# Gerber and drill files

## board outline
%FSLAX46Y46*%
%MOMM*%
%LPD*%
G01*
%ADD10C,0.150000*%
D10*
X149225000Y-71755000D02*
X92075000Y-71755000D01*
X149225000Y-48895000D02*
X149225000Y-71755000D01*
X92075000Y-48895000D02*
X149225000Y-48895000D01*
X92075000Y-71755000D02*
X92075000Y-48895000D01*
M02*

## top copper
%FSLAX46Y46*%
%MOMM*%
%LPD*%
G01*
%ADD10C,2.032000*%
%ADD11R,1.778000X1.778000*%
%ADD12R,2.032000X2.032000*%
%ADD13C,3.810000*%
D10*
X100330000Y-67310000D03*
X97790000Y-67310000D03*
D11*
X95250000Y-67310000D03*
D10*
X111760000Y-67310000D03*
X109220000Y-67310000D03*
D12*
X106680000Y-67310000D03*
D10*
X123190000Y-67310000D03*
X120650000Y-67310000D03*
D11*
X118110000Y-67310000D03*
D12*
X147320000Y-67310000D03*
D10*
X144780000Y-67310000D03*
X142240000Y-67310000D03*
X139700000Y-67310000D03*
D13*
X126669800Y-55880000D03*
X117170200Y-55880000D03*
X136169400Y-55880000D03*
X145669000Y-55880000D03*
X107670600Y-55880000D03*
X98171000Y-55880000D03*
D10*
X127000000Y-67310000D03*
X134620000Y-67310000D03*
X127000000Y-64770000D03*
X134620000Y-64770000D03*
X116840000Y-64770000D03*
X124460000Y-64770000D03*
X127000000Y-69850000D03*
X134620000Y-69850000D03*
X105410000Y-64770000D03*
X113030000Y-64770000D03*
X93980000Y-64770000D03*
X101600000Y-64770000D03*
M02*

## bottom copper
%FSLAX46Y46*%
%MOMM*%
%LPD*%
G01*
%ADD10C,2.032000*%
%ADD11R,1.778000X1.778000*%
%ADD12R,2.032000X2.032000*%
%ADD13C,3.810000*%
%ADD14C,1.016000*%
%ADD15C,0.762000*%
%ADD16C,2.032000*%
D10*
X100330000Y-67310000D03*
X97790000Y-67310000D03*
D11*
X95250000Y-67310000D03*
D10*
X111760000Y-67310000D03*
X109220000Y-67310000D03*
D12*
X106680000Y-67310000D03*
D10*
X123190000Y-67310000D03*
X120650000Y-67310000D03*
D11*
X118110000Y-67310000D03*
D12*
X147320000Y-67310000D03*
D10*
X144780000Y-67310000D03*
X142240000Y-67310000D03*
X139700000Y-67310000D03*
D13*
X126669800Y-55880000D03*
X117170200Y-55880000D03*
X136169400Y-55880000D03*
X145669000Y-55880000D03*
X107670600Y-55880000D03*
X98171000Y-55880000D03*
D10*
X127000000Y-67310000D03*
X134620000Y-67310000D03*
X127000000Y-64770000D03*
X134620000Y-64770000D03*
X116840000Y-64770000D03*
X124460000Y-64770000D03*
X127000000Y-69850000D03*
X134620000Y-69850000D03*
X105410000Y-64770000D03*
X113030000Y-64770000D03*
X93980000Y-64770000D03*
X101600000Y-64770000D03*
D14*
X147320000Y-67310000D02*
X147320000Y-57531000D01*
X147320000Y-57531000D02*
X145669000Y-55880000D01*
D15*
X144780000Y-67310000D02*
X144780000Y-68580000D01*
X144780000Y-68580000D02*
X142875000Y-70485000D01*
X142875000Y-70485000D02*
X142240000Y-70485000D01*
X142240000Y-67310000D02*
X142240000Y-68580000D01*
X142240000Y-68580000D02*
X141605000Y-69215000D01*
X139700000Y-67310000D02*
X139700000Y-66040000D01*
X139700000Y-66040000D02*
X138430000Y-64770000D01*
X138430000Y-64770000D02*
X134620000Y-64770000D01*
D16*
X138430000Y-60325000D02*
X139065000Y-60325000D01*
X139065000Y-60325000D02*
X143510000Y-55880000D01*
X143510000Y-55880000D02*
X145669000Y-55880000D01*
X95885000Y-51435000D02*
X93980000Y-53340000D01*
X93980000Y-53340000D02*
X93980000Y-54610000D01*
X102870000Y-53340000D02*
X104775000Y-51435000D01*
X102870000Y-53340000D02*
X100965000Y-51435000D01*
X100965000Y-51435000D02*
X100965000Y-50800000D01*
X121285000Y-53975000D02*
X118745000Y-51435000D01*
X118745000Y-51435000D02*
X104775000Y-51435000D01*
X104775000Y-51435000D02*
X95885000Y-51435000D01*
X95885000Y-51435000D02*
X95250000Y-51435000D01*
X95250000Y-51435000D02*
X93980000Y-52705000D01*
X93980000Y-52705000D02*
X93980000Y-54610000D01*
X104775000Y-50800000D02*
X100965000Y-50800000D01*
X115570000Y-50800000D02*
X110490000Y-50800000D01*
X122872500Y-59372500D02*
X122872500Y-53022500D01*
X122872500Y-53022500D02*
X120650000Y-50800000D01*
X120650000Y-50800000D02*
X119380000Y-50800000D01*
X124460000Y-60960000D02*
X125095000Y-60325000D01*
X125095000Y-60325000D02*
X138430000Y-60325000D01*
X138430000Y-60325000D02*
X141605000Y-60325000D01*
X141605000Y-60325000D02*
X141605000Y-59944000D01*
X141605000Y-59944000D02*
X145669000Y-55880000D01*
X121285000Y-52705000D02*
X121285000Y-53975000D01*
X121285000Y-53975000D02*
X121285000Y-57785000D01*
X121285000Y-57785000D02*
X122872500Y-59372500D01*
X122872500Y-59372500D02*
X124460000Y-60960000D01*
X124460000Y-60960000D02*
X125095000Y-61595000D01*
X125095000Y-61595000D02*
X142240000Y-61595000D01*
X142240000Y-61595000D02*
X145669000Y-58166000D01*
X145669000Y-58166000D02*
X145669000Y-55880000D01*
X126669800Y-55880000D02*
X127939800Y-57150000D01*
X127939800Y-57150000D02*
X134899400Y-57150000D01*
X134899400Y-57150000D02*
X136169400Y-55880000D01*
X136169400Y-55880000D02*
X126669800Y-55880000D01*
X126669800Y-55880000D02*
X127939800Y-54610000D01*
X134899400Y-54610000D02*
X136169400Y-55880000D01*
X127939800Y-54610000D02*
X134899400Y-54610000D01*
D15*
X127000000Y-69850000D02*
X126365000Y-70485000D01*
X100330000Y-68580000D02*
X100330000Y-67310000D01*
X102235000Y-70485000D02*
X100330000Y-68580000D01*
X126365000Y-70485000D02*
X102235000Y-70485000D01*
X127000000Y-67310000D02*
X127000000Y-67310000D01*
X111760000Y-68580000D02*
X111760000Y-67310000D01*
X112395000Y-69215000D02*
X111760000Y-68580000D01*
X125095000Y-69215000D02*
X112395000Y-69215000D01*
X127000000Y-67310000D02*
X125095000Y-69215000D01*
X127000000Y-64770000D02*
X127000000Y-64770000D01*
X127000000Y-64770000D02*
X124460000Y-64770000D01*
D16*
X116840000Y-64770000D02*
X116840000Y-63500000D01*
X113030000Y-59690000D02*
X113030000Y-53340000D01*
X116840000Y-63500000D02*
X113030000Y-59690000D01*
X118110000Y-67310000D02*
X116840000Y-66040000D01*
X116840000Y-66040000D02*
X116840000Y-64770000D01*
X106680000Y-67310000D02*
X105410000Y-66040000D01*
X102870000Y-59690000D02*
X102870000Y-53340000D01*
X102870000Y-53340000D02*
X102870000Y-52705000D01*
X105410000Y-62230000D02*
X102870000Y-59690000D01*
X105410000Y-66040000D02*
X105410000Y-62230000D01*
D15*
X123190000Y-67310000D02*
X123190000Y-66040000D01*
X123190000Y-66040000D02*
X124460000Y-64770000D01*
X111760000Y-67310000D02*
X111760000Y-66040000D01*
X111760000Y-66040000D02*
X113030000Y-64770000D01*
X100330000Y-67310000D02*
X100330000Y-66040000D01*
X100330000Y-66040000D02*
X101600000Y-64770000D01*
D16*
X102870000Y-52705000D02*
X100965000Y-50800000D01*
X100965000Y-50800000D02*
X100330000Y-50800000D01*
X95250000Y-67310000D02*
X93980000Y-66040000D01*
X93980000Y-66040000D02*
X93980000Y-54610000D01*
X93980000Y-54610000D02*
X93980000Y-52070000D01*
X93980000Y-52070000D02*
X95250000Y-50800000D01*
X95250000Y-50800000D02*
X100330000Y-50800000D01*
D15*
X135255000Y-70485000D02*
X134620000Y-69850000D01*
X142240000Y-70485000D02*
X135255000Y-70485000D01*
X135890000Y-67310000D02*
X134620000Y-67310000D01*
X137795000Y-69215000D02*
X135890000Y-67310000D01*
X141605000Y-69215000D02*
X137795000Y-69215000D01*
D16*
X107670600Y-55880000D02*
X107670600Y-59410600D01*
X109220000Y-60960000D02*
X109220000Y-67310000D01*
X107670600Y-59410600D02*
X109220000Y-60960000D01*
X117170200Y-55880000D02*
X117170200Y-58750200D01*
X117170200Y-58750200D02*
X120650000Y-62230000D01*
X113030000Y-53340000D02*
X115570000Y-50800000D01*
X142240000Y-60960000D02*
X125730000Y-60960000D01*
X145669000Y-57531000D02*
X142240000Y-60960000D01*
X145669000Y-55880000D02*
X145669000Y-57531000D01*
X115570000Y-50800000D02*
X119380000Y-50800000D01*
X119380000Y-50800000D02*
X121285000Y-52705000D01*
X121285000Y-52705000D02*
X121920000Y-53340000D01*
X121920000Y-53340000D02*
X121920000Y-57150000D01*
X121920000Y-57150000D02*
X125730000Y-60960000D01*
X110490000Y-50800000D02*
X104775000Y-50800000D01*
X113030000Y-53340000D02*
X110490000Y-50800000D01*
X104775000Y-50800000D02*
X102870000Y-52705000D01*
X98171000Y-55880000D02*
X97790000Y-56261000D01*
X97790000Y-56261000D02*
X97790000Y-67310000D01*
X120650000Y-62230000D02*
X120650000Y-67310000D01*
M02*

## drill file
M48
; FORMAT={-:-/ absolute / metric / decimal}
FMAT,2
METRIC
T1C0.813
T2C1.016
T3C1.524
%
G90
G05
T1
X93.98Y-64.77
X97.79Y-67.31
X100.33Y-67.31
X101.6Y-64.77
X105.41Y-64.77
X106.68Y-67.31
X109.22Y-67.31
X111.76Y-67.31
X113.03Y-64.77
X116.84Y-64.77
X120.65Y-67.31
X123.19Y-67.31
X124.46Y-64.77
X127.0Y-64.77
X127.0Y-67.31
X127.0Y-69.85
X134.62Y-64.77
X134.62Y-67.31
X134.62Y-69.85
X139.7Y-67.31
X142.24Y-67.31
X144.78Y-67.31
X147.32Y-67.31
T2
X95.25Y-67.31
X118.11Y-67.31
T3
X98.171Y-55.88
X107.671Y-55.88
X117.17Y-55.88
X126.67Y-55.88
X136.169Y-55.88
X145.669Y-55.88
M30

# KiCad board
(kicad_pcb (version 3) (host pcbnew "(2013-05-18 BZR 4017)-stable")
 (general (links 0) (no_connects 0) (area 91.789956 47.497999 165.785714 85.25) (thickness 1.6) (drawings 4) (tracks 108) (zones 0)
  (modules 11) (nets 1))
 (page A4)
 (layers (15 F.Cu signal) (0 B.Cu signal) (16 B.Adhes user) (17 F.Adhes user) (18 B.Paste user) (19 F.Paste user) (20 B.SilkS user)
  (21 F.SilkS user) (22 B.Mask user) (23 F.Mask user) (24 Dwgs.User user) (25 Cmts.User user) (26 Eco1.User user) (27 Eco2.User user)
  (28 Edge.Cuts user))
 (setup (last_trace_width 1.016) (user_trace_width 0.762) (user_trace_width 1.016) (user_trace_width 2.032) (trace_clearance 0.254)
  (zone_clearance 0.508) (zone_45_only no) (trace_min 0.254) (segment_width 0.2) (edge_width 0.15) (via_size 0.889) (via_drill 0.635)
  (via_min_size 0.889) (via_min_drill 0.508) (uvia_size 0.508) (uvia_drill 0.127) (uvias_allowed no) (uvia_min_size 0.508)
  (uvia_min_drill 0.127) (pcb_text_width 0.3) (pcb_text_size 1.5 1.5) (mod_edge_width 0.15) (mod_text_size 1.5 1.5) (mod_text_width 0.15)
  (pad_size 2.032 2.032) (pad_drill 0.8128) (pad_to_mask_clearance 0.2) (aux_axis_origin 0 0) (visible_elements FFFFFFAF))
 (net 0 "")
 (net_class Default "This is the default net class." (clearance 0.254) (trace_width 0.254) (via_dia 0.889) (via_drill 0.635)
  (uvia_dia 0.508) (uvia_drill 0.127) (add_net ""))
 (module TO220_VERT (layer F.Cu) (at 97.79 67.31 270)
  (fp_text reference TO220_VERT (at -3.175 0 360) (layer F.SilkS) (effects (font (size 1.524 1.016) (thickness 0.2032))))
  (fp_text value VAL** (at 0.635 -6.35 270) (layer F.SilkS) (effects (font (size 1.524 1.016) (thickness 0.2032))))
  (pad 2 thru_hole circle (at 0 -2.54 270) (size 2.032 2.032) (drill 0.8128) (layers *.Cu *.Mask F.SilkS))
  (pad 3 thru_hole circle (at 0 0 270) (size 2.032 2.032) (drill 0.8128) (layers *.Cu *.Mask F.SilkS))
  (pad 1 thru_hole rect (at 0 2.54 270) (size 1.778 1.778) (drill 1.016) (layers *.Cu *.Mask F.SilkS)))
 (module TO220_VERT (layer F.Cu) (at 109.22 67.31 270)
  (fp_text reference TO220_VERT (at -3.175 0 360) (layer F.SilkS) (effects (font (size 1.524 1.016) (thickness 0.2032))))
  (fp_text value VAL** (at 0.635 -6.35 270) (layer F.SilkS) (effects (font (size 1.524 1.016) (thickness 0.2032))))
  (pad 2 thru_hole circle (at 0 -2.54 270) (size 2.032 2.032) (drill 0.8128) (layers *.Cu *.Mask F.SilkS))
  (pad 3 thru_hole circle (at 0 0 270) (size 2.032 2.032) (drill 0.8128) (layers *.Cu *.Mask F.SilkS))
  (pad 1 thru_hole rect (at 0 2.54 270) (size 2.032 2.032) (drill 0.8128) (layers *.Cu *.Mask F.SilkS)))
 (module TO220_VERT (layer F.Cu) (at 120.65 67.31 270)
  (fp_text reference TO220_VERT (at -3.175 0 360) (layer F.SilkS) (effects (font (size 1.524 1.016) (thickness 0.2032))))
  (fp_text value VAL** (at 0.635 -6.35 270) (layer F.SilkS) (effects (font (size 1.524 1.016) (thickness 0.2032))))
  (pad 2 thru_hole circle (at 0 -2.54 270) (size 2.032 2.032) (drill 0.8128) (layers *.Cu *.Mask F.SilkS))
  (pad 3 thru_hole circle (at 0 0 270) (size 2.032 2.032) (drill 0.8128) (layers *.Cu *.Mask F.SilkS))
  (pad 1 thru_hole rect (at 0 2.54 270) (size 1.778 1.778) (drill 1.016) (layers *.Cu *.Mask F.SilkS)))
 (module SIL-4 (layer F.Cu) (at 143.51 67.31 180)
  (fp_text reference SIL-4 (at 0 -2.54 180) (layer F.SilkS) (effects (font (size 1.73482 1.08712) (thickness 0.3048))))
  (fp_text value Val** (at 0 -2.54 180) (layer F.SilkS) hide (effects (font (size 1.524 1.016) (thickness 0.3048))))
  (pad 1 thru_hole rect (at -3.81 0 180) (size 2.032 2.032) (drill 0.8128) (layers *.Cu *.Mask F.SilkS))
  (pad 2 thru_hole circle (at -1.27 0 180) (size 2.032 2.032) (drill 0.8128) (layers *.Cu *.Mask F.SilkS))
  (pad 3 thru_hole circle (at 1.27 0 180) (size 2.032 2.032) (drill 0.8128) (layers *.Cu *.Mask F.SilkS))
  (pad 4 thru_hole circle (at 3.81 0 180) (size 2.032 2.032) (drill 0.8128) (layers *.Cu *.Mask F.SilkS)))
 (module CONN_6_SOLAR (layer F.Cu) (at 121.92 55.88)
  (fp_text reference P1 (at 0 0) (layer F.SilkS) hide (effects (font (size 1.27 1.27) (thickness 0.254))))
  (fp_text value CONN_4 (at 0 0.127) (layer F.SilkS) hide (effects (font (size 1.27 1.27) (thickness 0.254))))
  (pad 4 thru_hole circle (at 4.7498 0) (size 3.81 3.81) (drill 1.524) (layers *.Cu *.Mask))
  (pad 3 thru_hole circle (at -4.7498 0) (size 3.81 3.81) (drill 1.524) (layers *.Cu *.Mask))
  (pad 5 thru_hole circle (at 14.2494 0) (size 3.81 3.81) (drill 1.524) (layers *.Cu *.Mask))
  (pad 6 thru_hole circle (at 23.749 0) (size 3.81 3.81) (drill 1.524) (layers *.Cu *.Mask))
  (pad 2 thru_hole circle (at -14.2494 0) (size 3.81 3.81) (drill 1.524) (layers *.Cu *.Mask))
  (pad 1 thru_hole circle (at -23.749 0) (size 3.81 3.81) (drill 1.524) (layers *.Cu *.Mask)))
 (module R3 (layer F.Cu) (at 130.81 67.31) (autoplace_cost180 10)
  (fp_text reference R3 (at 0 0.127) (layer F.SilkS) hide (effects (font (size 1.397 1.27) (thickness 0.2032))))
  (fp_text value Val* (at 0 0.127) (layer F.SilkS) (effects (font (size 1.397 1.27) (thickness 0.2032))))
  (pad 1 thru_hole circle (at -3.81 0) (size 2.032 2.032) (drill 0.8128) (layers *.Cu *.Mask F.SilkS))
  (pad 2 thru_hole circle (at 3.81 0) (size 2.032 2.032) (drill 0.8128) (layers *.Cu *.Mask F.SilkS)))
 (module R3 (layer F.Cu) (at 130.81 64.77) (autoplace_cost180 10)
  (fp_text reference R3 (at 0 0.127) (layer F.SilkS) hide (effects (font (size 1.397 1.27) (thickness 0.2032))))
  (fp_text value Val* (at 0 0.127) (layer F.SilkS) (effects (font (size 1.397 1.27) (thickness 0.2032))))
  (pad 1 thru_hole circle (at -3.81 0) (size 2.032 2.032) (drill 0.8128) (layers *.Cu *.Mask F.SilkS))
  (pad 2 thru_hole circle (at 3.81 0) (size 2.032 2.032) (drill 0.8128) (layers *.Cu *.Mask F.SilkS)))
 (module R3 (layer F.Cu) (at 120.65 64.77) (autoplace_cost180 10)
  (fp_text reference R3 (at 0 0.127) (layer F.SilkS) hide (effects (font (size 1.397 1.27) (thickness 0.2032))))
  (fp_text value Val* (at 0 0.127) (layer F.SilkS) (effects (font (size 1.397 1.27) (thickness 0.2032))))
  (pad 1 thru_hole circle (at -3.81 0) (size 2.032 2.032) (drill 0.8128) (layers *.Cu *.Mask F.SilkS))
  (pad 2 thru_hole circle (at 3.81 0) (size 2.032 2.032) (drill 0.8128) (layers *.Cu *.Mask F.SilkS)))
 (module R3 (layer F.Cu) (at 130.81 69.85) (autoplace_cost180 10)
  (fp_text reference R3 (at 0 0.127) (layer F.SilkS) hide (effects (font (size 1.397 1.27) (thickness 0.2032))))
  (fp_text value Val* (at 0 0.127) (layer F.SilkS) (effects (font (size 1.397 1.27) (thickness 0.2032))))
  (pad 1 thru_hole circle (at -3.81 0) (size 2.032 2.032) (drill 0.8128) (layers *.Cu *.Mask F.SilkS))
  (pad 2 thru_hole circle (at 3.81 0) (size 2.032 2.032) (drill 0.8128) (layers *.Cu *.Mask F.SilkS)))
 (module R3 (layer F.Cu) (at 109.22 64.77) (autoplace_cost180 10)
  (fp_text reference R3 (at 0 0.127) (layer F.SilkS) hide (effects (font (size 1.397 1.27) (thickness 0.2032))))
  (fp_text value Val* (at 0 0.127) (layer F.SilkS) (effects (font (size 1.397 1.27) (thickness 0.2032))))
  (pad 1 thru_hole circle (at -3.81 0) (size 2.032 2.032) (drill 0.8128) (layers *.Cu *.Mask F.SilkS))
  (pad 2 thru_hole circle (at 3.81 0) (size 2.032 2.032) (drill 0.8128) (layers *.Cu *.Mask F.SilkS)))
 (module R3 (layer F.Cu) (at 97.79 64.77) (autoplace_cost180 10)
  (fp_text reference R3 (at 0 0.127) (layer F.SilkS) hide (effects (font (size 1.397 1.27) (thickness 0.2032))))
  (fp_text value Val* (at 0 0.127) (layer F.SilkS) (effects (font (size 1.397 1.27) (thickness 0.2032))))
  (pad 1 thru_hole circle (at -3.81 0) (size 2.032 2.032) (drill 0.8128) (layers *.Cu *.Mask F.SilkS))
  (pad 2 thru_hole circle (at 3.81 0) (size 2.032 2.032) (drill 0.8128) (layers *.Cu *.Mask F.SilkS)))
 (gr_line (start 149.225 71.755) (end 92.075 71.755) (angle 90) (layer Edge.Cuts) (width 0.15))
 (gr_line (start 149.225 48.895) (end 149.225 71.755) (angle 90) (layer Edge.Cuts) (width 0.15))
 (gr_line (start 92.075 48.895) (end 149.225 48.895) (angle 90) (layer Edge.Cuts) (width 0.15))
 (gr_line (start 92.075 71.755) (end 92.075 48.895) (angle 90) (layer Edge.Cuts) (width 0.15))
 (segment (start 147.32 67.31) (end 147.32 57.531) (width 1.016) (layer B.Cu) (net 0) (status 400000))
 (segment (start 147.32 57.531) (end 145.669 55.88) (width 1.016) (layer B.Cu) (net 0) (status 800000))
 (segment (start 144.78 67.31) (end 144.78 68.58) (width 0.762) (layer B.Cu) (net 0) (status 400000))
 (segment (start 144.78 68.58) (end 142.875 70.485) (width 0.762) (layer B.Cu) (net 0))
 (segment (start 142.875 70.485) (end 142.24 70.485) (width 0.762) (layer B.Cu) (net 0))
 (segment (start 142.24 67.31) (end 142.24 68.58) (width 0.762) (layer B.Cu) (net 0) (status 400000))
 (segment (start 142.24 68.58) (end 141.605 69.215) (width 0.762) (layer B.Cu) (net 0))
 (segment (start 139.7 67.31) (end 139.7 66.04) (width 0.762) (layer B.Cu) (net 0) (status 400000))
 (segment (start 139.7 66.04) (end 138.43 64.77) (width 0.762) (layer B.Cu) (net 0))
 (segment (start 138.43 64.77) (end 134.62 64.77) (width 0.762) (layer B.Cu) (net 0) (status 800000))
 (segment (start 138.43 60.325) (end 139.065 60.325) (width 2.032) (layer B.Cu) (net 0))
 (segment (start 139.065 60.325) (end 143.51 55.88) (width 2.032) (layer B.Cu) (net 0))
 (segment (start 143.51 55.88) (end 145.669 55.88) (width 2.032) (layer B.Cu) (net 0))
 (segment (start 95.885 51.435) (end 93.98 53.34) (width 2.032) (layer B.Cu) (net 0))
 (segment (start 93.98 53.34) (end 93.98 54.61) (width 2.032) (layer B.Cu) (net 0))
 (segment (start 102.87 53.34) (end 104.775 51.435) (width 2.032) (layer B.Cu) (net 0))
 (segment (start 102.87 53.34) (end 100.965 51.435) (width 2.032) (layer B.Cu) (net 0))
 (segment (start 100.965 51.435) (end 100.965 50.8) (width 2.032) (layer B.Cu) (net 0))
 (segment (start 121.285 53.975) (end 118.745 51.435) (width 2.032) (layer B.Cu) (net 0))
 (segment (start 118.745 51.435) (end 104.775 51.435) (width 2.032) (layer B.Cu) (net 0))
 (segment (start 104.775 51.435) (end 95.885 51.435) (width 2.032) (layer B.Cu) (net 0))
 (segment (start 95.885 51.435) (end 95.25 51.435) (width 2.032) (layer B.Cu) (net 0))
 (segment (start 95.25 51.435) (end 93.98 52.705) (width 2.032) (layer B.Cu) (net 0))
 (segment (start 93.98 52.705) (end 93.98 54.61) (width 2.032) (layer B.Cu) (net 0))
 (segment (start 104.775 50.8) (end 100.965 50.8) (width 2.032) (layer B.Cu) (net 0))
 (segment (start 115.57 50.8) (end 110.49 50.8) (width 2.032) (layer B.Cu) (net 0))
 (segment (start 122.8725 59.3725) (end 122.8725 53.0225) (width 2.032) (layer B.Cu) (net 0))
 (segment (start 122.8725 53.0225) (end 120.65 50.8) (width 2.032) (layer B.Cu) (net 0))
 (segment (start 120.65 50.8) (end 119.38 50.8) (width 2.032) (layer B.Cu) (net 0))
 (segment (start 124.46 60.96) (end 125.095 60.325) (width 2.032) (layer B.Cu) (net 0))
 (segment (start 125.095 60.325) (end 138.43 60.325) (width 2.032) (layer B.Cu) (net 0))
 (segment (start 138.43 60.325) (end 141.605 60.325) (width 2.032) (layer B.Cu) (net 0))
 (segment (start 141.605 60.325) (end 141.605 59.944) (width 2.032) (layer B.Cu) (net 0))
 (segment (start 141.605 59.944) (end 145.669 55.88) (width 2.032) (layer B.Cu) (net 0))
 (segment (start 121.285 52.705) (end 121.285 53.975) (width 2.032) (layer B.Cu) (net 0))
 (segment (start 121.285 53.975) (end 121.285 57.785) (width 2.032) (layer B.Cu) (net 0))
 (segment (start 121.285 57.785) (end 122.8725 59.3725) (width 2.032) (layer B.Cu) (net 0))
 (segment (start 122.8725 59.3725) (end 124.46 60.96) (width 2.032) (layer B.Cu) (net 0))
 (segment (start 124.46 60.96) (end 125.095 61.595) (width 2.032) (layer B.Cu) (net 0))
 (segment (start 125.095 61.595) (end 142.24 61.595) (width 2.032) (layer B.Cu) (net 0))
 (segment (start 142.24 61.595) (end 145.669 58.166) (width 2.032) (layer B.Cu) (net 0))
 (segment (start 145.669 58.166) (end 145.669 55.88) (width 2.032) (layer B.Cu) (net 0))
 (segment (start 126.6698 55.88) (end 127.9398 57.15) (width 2.032) (layer B.Cu) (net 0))
 (segment (start 127.9398 57.15) (end 134.8994 57.15) (width 2.032) (layer B.Cu) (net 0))
 (segment (start 134.8994 57.15) (end 136.1694 55.88) (width 2.032) (layer B.Cu) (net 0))
 (segment (start 136.1694 55.88) (end 126.6698 55.88) (width 2.032) (layer B.Cu) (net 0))
 (segment (start 126.6698 55.88) (end 127.9398 54.61) (width 2.032) (layer B.Cu) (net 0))
 (segment (start 134.8994 54.61) (end 136.1694 55.88) (width 2.032) (layer B.Cu) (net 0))
 (segment (start 127.9398 54.61) (end 134.8994 54.61) (width 2.032) (layer B.Cu) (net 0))
 (segment (start 127 69.85) (end 126.365 70.485) (width 0.762) (layer B.Cu) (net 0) (status 30))
 (segment (start 100.33 68.58) (end 100.33 67.31) (width 0.762) (layer B.Cu) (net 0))
 (segment (start 102.235 70.485) (end 100.33 68.58) (width 0.762) (layer B.Cu) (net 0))
 (segment (start 126.365 70.485) (end 102.235 70.485) (width 0.762) (layer B.Cu) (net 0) (status 10))
 (segment (start 127 67.31) (end 127 67.31) (width 0.762) (layer B.Cu) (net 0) (status 10))
 (segment (start 111.76 68.58) (end 111.76 67.31) (width 0.762) (layer B.Cu) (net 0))
 (segment (start 112.395 69.215) (end 111.76 68.58) (width 0.762) (layer B.Cu) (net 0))
 (segment (start 125.095 69.215) (end 112.395 69.215) (width 0.762) (layer B.Cu) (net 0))
 (segment (start 127 67.31) (end 125.095 69.215) (width 0.762) (layer B.Cu) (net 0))
 (segment (start 127 64.77) (end 127 64.77) (width 0.762) (layer B.Cu) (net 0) (status 10))
 (segment (start 127 64.77) (end 124.46 64.77) (width 0.762) (layer B.Cu) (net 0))
 (segment (start 116.84 64.77) (end 116.84 63.5) (width 2.032) (layer B.Cu) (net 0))
 (segment (start 113.03 59.69) (end 113.03 53.34) (width 2.032) (layer B.Cu) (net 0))
 (segment (start 116.84 63.5) (end 113.03 59.69) (width 2.032) (layer B.Cu) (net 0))
 (segment (start 118.11 67.31) (end 116.84 66.04) (width 2.032) (layer B.Cu) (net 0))
 (segment (start 116.84 66.04) (end 116.84 64.77) (width 2.032) (layer B.Cu) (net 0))
 (segment (start 106.68 67.31) (end 105.41 66.04) (width 2.032) (layer B.Cu) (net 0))
 (segment (start 102.87 59.69) (end 102.87 53.34) (width 2.032) (layer B.Cu) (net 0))
 (segment (start 102.87 53.34) (end 102.87 52.705) (width 2.032) (layer B.Cu) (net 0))
 (segment (start 105.41 62.23) (end 102.87 59.69) (width 2.032) (layer B.Cu) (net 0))
 (segment (start 105.41 66.04) (end 105.41 62.23) (width 2.032) (layer B.Cu) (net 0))
 (segment (start 123.19 67.31) (end 123.19 66.04) (width 0.762) (layer B.Cu) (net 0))
 (segment (start 123.19 66.04) (end 124.46 64.77) (width 0.762) (layer B.Cu) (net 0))
 (segment (start 111.76 67.31) (end 111.76 66.04) (width 0.762) (layer B.Cu) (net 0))
 (segment (start 111.76 66.04) (end 113.03 64.77) (width 0.762) (layer B.Cu) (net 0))
 (segment (start 100.33 67.31) (end 100.33 66.04) (width 0.762) (layer B.Cu) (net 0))
 (segment (start 100.33 66.04) (end 101.6 64.77) (width 0.762) (layer B.Cu) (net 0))
 (segment (start 102.87 52.705) (end 100.965 50.8) (width 2.032) (layer B.Cu) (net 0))
 (segment (start 100.965 50.8) (end 100.33 50.8) (width 2.032) (layer B.Cu) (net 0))
 (segment (start 95.25 67.31) (end 93.98 66.04) (width 2.032) (layer B.Cu) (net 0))
 (segment (start 93.98 66.04) (end 93.98 54.61) (width 2.032) (layer B.Cu) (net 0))
 (segment (start 93.98 54.61) (end 93.98 52.07) (width 2.032) (layer B.Cu) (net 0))
 (segment (start 93.98 52.07) (end 95.25 50.8) (width 2.032) (layer B.Cu) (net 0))
 (segment (start 95.25 50.8) (end 100.33 50.8) (width 2.032) (layer B.Cu) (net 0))
 (segment (start 135.255 70.485) (end 134.62 69.85) (width 0.762) (layer B.Cu) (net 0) (status 30))
 (segment (start 142.24 70.485) (end 135.255 70.485) (width 0.762) (layer B.Cu) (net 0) (status 20))
 (segment (start 135.89 67.31) (end 134.62 67.31) (width 0.762) (layer B.Cu) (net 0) (status 20))
 (segment (start 137.795 69.215) (end 135.89 67.31) (width 0.762) (layer B.Cu) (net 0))
 (segment (start 141.605 69.215) (end 137.795 69.215) (width 0.762) (layer B.Cu) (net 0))
 (segment (start 107.6706 55.88) (end 107.6706 59.4106) (width 2.032) (layer B.Cu) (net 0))
 (segment (start 109.22 60.96) (end 109.22 67.31) (width 2.032) (layer B.Cu) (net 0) (status 20))
 (segment (start 107.6706 59.4106) (end 109.22 60.96) (width 2.032) (layer B.Cu) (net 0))
 (segment (start 117.1702 55.88) (end 117.1702 58.7502) (width 2.032) (layer B.Cu) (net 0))
 (segment (start 117.1702 58.7502) (end 120.65 62.23) (width 2.032) (layer B.Cu) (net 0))
 (segment (start 113.03 53.34) (end 115.57 50.8) (width 2.032) (layer B.Cu) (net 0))
 (segment (start 142.24 60.96) (end 125.73 60.96) (width 2.032) (layer B.Cu) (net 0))
 (segment (start 145.669 57.531) (end 142.24 60.96) (width 2.032) (layer B.Cu) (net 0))
 (segment (start 145.669 55.88) (end 145.669 57.531) (width 2.032) (layer B.Cu) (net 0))
 (segment (start 115.57 50.8) (end 119.38 50.8) (width 2.032) (layer B.Cu) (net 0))
 (segment (start 119.38 50.8) (end 121.285 52.705) (width 2.032) (layer B.Cu) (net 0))
 (segment (start 121.285 52.705) (end 121.92 53.34) (width 2.032) (layer B.Cu) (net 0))
 (segment (start 121.92 53.34) (end 121.92 57.15) (width 2.032) (layer B.Cu) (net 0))
 (segment (start 121.92 57.15) (end 125.73 60.96) (width 2.032) (layer B.Cu) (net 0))
 (segment (start 110.49 50.8) (end 104.775 50.8) (width 2.032) (layer B.Cu) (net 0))
 (segment (start 113.03 53.34) (end 110.49 50.8) (width 2.032) (layer B.Cu) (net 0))
 (segment (start 104.775 50.8) (end 102.87 52.705) (width 2.032) (layer B.Cu) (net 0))
 (segment (start 98.171 55.88) (end 97.79 56.261) (width 2.032) (layer B.Cu) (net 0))
 (segment (start 97.79 56.261) (end 97.79 67.31) (width 2.032) (layer B.Cu) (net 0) (status 20))
 (segment (start 120.65 62.23) (end 120.65 67.31) (width 2.032) (layer B.Cu) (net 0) (status 20)))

